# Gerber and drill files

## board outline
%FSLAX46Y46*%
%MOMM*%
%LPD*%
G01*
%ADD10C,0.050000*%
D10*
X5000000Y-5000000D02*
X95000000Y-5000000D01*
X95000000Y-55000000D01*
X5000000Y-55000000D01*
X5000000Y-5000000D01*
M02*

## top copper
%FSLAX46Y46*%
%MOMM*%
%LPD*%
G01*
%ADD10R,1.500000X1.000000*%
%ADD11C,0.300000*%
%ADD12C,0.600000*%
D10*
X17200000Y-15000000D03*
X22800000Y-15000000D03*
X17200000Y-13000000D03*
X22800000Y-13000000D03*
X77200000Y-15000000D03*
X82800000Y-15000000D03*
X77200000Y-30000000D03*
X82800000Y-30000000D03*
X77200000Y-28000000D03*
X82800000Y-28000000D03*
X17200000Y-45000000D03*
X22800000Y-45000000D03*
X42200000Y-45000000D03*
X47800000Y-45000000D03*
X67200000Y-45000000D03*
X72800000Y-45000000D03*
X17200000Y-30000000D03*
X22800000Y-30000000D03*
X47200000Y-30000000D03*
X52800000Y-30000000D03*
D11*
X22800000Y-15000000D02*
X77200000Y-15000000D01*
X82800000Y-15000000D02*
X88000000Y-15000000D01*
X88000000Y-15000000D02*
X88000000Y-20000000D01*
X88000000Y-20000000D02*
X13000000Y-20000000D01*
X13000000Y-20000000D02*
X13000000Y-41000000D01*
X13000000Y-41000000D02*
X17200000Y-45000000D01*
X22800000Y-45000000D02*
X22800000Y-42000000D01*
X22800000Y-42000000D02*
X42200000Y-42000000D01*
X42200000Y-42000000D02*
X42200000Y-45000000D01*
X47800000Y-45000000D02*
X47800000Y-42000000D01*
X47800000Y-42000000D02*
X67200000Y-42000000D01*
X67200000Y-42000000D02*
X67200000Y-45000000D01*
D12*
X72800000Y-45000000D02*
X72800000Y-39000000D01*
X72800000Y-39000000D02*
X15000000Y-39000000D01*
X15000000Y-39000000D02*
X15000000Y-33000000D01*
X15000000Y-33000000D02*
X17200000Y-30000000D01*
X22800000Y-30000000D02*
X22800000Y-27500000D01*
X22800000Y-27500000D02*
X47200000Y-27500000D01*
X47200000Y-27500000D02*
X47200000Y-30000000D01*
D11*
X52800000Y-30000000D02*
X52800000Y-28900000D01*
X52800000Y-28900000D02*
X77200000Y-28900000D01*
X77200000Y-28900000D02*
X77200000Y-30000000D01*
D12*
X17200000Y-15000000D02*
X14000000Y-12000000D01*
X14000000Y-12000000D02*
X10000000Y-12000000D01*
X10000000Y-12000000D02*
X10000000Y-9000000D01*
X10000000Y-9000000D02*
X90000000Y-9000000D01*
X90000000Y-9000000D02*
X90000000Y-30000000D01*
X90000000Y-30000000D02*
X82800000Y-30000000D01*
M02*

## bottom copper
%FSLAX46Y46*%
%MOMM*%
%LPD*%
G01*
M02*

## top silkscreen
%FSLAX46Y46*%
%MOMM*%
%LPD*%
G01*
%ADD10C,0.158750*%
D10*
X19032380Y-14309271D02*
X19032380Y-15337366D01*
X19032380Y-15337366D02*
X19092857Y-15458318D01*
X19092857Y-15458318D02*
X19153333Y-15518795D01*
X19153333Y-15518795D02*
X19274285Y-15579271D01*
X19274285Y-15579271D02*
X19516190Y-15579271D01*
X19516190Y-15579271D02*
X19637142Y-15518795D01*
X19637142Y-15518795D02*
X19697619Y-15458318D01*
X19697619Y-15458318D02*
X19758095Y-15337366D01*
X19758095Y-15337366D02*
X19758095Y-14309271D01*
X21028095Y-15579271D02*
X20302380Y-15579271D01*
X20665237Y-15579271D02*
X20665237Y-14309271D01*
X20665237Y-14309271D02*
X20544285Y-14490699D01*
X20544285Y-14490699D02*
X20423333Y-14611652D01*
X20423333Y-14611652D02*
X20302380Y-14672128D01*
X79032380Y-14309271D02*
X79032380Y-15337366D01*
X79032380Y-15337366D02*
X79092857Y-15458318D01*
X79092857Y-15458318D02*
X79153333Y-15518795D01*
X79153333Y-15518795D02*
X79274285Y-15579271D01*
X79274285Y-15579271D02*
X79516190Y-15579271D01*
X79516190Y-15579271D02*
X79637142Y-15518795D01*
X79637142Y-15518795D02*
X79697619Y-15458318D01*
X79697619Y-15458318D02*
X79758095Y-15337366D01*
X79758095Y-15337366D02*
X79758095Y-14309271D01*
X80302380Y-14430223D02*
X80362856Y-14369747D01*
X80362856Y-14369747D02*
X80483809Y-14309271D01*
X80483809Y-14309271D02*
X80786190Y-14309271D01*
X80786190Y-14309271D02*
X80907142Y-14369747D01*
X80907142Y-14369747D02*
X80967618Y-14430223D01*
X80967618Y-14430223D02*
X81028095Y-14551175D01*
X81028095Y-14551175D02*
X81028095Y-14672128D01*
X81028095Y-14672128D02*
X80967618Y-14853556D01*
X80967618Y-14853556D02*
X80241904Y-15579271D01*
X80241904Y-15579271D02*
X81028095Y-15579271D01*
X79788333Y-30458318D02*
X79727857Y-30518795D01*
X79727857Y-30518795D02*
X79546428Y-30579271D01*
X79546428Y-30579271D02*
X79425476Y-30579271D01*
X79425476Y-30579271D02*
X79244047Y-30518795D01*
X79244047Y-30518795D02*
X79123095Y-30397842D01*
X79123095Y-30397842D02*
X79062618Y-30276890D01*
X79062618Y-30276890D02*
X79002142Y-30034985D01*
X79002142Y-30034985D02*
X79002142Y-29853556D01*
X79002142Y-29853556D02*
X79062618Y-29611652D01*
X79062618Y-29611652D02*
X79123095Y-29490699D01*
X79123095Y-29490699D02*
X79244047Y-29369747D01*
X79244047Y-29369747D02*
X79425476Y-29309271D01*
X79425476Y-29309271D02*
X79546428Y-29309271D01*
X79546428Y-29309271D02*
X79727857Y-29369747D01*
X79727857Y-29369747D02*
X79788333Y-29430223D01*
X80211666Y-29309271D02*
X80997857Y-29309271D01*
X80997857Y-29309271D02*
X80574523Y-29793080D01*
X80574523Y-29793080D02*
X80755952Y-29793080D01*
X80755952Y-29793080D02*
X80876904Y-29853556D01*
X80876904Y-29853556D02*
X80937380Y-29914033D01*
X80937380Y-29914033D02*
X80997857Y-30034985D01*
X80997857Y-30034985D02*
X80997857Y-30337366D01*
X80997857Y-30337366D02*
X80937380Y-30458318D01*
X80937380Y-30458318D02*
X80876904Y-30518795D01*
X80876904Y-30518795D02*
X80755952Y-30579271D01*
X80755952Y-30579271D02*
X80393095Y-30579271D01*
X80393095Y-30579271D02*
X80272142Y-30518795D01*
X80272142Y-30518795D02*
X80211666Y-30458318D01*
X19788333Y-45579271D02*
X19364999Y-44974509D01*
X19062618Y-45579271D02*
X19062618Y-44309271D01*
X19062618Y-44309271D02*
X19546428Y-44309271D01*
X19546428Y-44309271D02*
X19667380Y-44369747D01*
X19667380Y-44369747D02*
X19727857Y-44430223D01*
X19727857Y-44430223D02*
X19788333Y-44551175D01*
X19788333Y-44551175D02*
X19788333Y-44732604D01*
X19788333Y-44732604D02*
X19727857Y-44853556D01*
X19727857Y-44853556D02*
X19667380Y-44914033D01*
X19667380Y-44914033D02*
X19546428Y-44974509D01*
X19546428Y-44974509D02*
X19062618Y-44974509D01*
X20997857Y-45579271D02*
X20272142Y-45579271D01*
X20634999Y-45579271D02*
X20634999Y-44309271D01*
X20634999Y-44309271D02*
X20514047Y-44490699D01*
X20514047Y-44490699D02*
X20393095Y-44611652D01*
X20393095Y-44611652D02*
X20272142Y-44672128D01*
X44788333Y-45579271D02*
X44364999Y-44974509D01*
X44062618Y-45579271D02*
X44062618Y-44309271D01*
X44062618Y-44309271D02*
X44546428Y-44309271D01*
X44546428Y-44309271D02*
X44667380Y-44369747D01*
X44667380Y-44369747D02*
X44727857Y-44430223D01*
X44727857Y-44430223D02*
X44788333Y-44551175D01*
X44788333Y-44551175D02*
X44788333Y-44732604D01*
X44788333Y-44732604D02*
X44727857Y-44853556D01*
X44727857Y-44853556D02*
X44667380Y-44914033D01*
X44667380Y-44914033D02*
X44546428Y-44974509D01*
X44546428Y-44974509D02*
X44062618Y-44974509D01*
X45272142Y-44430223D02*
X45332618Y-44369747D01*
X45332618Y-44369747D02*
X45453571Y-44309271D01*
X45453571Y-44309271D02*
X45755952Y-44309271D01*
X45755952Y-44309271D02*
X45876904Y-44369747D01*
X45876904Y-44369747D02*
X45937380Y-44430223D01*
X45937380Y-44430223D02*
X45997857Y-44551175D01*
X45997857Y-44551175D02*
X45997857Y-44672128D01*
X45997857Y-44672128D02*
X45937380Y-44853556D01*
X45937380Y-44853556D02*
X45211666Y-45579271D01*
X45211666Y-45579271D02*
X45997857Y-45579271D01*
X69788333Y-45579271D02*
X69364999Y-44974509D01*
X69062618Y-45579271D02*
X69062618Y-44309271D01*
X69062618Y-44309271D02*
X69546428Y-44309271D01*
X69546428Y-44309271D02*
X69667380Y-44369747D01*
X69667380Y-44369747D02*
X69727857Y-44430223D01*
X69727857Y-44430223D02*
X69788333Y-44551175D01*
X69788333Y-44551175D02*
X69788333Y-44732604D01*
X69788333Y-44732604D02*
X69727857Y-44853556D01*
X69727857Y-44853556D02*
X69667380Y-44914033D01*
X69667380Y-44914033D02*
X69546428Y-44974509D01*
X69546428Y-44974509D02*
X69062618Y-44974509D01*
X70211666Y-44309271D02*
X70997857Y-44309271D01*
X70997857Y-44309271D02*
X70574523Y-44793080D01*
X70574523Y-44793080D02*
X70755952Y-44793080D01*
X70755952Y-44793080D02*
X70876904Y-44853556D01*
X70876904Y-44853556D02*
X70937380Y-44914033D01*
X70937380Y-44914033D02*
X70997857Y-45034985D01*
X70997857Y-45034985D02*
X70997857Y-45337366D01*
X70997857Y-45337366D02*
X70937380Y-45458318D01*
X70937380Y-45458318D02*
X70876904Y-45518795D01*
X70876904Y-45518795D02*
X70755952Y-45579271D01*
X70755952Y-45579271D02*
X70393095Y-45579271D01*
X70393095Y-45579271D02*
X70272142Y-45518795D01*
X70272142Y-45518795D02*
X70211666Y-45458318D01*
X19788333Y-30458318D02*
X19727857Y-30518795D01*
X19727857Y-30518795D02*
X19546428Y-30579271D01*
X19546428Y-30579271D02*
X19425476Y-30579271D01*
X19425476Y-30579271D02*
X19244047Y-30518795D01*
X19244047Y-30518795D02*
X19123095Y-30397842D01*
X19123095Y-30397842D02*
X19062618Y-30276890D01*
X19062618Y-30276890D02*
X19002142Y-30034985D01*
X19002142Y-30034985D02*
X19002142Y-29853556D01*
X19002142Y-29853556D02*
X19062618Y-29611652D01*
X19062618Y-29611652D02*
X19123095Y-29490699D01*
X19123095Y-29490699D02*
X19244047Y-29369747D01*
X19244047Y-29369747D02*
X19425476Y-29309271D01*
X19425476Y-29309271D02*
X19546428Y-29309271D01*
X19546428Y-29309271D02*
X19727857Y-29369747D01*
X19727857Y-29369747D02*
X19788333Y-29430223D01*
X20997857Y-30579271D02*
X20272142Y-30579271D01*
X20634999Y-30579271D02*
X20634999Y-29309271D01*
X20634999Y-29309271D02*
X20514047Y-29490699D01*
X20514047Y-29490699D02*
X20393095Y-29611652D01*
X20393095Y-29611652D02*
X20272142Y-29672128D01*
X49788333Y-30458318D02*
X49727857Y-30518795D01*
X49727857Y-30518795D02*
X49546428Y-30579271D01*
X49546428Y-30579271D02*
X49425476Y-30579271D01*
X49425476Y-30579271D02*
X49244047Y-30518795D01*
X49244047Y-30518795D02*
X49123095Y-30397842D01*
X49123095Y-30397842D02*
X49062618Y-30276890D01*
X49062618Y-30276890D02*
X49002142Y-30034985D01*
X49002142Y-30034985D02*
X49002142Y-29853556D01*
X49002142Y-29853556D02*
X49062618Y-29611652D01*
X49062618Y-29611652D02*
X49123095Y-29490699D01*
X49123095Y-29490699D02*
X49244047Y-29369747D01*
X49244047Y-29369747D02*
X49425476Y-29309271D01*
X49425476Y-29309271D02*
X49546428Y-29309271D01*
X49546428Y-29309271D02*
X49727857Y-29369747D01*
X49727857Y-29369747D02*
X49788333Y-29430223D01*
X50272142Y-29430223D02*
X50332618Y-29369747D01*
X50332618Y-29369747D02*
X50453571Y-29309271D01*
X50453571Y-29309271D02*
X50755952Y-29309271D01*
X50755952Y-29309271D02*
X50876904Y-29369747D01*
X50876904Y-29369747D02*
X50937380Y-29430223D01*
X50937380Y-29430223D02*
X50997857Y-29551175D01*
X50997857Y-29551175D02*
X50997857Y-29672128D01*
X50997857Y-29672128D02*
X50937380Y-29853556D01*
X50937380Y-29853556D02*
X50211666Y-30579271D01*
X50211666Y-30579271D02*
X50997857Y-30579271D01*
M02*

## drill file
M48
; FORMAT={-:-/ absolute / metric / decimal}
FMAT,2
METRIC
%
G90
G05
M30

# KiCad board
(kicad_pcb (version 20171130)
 (gr_rect (start 5 5) (end 95 55) (layer "Edge.Cuts") (width 0.05)) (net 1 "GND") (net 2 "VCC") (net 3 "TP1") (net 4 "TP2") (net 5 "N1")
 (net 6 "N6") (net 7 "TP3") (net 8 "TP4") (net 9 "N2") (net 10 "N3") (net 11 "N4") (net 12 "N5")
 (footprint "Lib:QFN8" (layer "F.Cu") (at 20 15 0) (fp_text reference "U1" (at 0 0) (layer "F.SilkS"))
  (pad "1" smd rect (at -2.8 0 0) (size 1.5 1.0) (layers "F.Cu" "F.Mask") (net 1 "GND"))
  (pad "2" smd rect (at 2.8 0 0) (size 1.5 1.0) (layers "F.Cu" "F.Mask") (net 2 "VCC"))
  (pad "3" smd rect (at -2.8 -2.0 0) (size 1.5 1.0) (layers "F.Cu" "F.Mask") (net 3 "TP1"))
  (pad "4" smd rect (at 2.8 -2.0 0) (size 1.5 1.0) (layers "F.Cu" "F.Mask") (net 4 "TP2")))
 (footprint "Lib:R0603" (layer "F.Cu") (at 80 15 0) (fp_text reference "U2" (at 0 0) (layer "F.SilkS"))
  (pad "1" smd rect (at -2.8 0 0) (size 1.5 1.0) (layers "F.Cu" "F.Mask") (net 2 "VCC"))
  (pad "2" smd rect (at 2.8 0 0) (size 1.5 1.0) (layers "F.Cu" "F.Mask") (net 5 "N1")))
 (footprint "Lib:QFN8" (layer "F.Cu") (at 80 30 0) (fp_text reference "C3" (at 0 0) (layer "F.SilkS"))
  (pad "1" smd rect (at -2.8 0 0) (size 1.5 1.0) (layers "F.Cu" "F.Mask") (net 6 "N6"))
  (pad "2" smd rect (at 2.8 0 0) (size 1.5 1.0) (layers "F.Cu" "F.Mask") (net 1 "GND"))
  (pad "3" smd rect (at -2.8 -2.0 0) (size 1.5 1.0) (layers "F.Cu" "F.Mask") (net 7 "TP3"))
  (pad "4" smd rect (at 2.8 -2.0 0) (size 1.5 1.0) (layers "F.Cu" "F.Mask") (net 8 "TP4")))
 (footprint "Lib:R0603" (layer "F.Cu") (at 20 45 0) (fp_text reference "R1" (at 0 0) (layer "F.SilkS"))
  (pad "1" smd rect (at -2.8 0 0) (size 1.5 1.0) (layers "F.Cu" "F.Mask") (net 5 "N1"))
  (pad "2" smd rect (at 2.8 0 0) (size 1.5 1.0) (layers "F.Cu" "F.Mask") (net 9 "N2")))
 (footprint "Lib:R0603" (layer "F.Cu") (at 45 45 0) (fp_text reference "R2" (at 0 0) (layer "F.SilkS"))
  (pad "1" smd rect (at -2.8 0 0) (size 1.5 1.0) (layers "F.Cu" "F.Mask") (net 9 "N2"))
  (pad "2" smd rect (at 2.8 0 0) (size 1.5 1.0) (layers "F.Cu" "F.Mask") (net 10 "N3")))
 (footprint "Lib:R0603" (layer "F.Cu") (at 70 45 0) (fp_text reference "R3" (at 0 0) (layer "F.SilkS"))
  (pad "1" smd rect (at -2.8 0 0) (size 1.5 1.0) (layers "F.Cu" "F.Mask") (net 10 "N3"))
  (pad "2" smd rect (at 2.8 0 0) (size 1.5 1.0) (layers "F.Cu" "F.Mask") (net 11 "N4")))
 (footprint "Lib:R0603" (layer "F.Cu") (at 20 30 0) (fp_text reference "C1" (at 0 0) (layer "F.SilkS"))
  (pad "1" smd rect (at -2.8 0 0) (size 1.5 1.0) (layers "F.Cu" "F.Mask") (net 11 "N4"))
  (pad "2" smd rect (at 2.8 0 0) (size 1.5 1.0) (layers "F.Cu" "F.Mask") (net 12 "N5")))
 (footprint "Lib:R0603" (layer "F.Cu") (at 50 30 0) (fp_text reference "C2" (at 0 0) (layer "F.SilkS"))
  (pad "1" smd rect (at -2.8 0 0) (size 1.5 1.0) (layers "F.Cu" "F.Mask") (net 12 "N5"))
  (pad "2" smd rect (at 2.8 0 0) (size 1.5 1.0) (layers "F.Cu" "F.Mask") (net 6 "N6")))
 (segment (start 22.8 15) (end 77.2 15) (width 0.3) (layer "F.Cu") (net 2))
 (segment (start 82.8 15) (end 88 15) (width 0.3) (layer "F.Cu") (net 5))
 (segment (start 88 15) (end 88 20) (width 0.3) (layer "F.Cu") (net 5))
 (segment (start 88 20) (end 13 20) (width 0.3) (layer "F.Cu") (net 5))
 (segment (start 13 20) (end 13 41) (width 0.3) (layer "F.Cu") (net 5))
 (segment (start 13 41) (end 17.2 45) (width 0.3) (layer "F.Cu") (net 5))
 (segment (start 22.8 45) (end 22.8 42) (width 0.3) (layer "F.Cu") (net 9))
 (segment (start 22.8 42) (end 42.2 42) (width 0.3) (layer "F.Cu") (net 9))
 (segment (start 42.2 42) (end 42.2 45) (width 0.3) (layer "F.Cu") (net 9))
 (segment (start 47.8 45) (end 47.8 42) (width 0.3) (layer "F.Cu") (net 10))
 (segment (start 47.8 42) (end 67.2 42) (width 0.3) (layer "F.Cu") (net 10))
 (segment (start 67.2 42) (end 67.2 45) (width 0.3) (layer "F.Cu") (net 10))
 (segment (start 72.8 45) (end 72.8 39) (width 0.6) (layer "F.Cu") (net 11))
 (segment (start 72.8 39) (end 15 39) (width 0.6) (layer "F.Cu") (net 11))
 (segment (start 15 39) (end 15 33) (width 0.6) (layer "F.Cu") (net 11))
 (segment (start 15 33) (end 17.2 30) (width 0.6) (layer "F.Cu") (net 11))
 (segment (start 22.8 30) (end 22.8 27.5) (width 0.6) (layer "F.Cu") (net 12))
 (segment (start 22.8 27.5) (end 47.2 27.5) (width 0.6) (layer "F.Cu") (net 12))
 (segment (start 47.2 27.5) (end 47.2 30) (width 0.6) (layer "F.Cu") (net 12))
 (segment (start 52.8 30) (end 52.8 28.9) (width 0.3) (layer "F.Cu") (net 6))
 (segment (start 52.8 28.9) (end 77.2 28.9) (width 0.3) (layer "F.Cu") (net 6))
 (segment (start 77.2 28.9) (end 77.2 30) (width 0.3) (layer "F.Cu") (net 6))
 (segment (start 17.2 15) (end 14 12) (width 0.6) (layer "F.Cu") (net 1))
 (segment (start 14 12) (end 10 12) (width 0.6) (layer "F.Cu") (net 1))
 (segment (start 10 12) (end 10 9) (width 0.6) (layer "F.Cu") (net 1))
 (segment (start 10 9) (end 90 9) (width 0.6) (layer "F.Cu") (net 1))
 (segment (start 90 9) (end 90 30) (width 0.6) (layer "F.Cu") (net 1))
 (segment (start 90 30) (end 82.8 30) (width 0.6) (layer "F.Cu") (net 1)))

